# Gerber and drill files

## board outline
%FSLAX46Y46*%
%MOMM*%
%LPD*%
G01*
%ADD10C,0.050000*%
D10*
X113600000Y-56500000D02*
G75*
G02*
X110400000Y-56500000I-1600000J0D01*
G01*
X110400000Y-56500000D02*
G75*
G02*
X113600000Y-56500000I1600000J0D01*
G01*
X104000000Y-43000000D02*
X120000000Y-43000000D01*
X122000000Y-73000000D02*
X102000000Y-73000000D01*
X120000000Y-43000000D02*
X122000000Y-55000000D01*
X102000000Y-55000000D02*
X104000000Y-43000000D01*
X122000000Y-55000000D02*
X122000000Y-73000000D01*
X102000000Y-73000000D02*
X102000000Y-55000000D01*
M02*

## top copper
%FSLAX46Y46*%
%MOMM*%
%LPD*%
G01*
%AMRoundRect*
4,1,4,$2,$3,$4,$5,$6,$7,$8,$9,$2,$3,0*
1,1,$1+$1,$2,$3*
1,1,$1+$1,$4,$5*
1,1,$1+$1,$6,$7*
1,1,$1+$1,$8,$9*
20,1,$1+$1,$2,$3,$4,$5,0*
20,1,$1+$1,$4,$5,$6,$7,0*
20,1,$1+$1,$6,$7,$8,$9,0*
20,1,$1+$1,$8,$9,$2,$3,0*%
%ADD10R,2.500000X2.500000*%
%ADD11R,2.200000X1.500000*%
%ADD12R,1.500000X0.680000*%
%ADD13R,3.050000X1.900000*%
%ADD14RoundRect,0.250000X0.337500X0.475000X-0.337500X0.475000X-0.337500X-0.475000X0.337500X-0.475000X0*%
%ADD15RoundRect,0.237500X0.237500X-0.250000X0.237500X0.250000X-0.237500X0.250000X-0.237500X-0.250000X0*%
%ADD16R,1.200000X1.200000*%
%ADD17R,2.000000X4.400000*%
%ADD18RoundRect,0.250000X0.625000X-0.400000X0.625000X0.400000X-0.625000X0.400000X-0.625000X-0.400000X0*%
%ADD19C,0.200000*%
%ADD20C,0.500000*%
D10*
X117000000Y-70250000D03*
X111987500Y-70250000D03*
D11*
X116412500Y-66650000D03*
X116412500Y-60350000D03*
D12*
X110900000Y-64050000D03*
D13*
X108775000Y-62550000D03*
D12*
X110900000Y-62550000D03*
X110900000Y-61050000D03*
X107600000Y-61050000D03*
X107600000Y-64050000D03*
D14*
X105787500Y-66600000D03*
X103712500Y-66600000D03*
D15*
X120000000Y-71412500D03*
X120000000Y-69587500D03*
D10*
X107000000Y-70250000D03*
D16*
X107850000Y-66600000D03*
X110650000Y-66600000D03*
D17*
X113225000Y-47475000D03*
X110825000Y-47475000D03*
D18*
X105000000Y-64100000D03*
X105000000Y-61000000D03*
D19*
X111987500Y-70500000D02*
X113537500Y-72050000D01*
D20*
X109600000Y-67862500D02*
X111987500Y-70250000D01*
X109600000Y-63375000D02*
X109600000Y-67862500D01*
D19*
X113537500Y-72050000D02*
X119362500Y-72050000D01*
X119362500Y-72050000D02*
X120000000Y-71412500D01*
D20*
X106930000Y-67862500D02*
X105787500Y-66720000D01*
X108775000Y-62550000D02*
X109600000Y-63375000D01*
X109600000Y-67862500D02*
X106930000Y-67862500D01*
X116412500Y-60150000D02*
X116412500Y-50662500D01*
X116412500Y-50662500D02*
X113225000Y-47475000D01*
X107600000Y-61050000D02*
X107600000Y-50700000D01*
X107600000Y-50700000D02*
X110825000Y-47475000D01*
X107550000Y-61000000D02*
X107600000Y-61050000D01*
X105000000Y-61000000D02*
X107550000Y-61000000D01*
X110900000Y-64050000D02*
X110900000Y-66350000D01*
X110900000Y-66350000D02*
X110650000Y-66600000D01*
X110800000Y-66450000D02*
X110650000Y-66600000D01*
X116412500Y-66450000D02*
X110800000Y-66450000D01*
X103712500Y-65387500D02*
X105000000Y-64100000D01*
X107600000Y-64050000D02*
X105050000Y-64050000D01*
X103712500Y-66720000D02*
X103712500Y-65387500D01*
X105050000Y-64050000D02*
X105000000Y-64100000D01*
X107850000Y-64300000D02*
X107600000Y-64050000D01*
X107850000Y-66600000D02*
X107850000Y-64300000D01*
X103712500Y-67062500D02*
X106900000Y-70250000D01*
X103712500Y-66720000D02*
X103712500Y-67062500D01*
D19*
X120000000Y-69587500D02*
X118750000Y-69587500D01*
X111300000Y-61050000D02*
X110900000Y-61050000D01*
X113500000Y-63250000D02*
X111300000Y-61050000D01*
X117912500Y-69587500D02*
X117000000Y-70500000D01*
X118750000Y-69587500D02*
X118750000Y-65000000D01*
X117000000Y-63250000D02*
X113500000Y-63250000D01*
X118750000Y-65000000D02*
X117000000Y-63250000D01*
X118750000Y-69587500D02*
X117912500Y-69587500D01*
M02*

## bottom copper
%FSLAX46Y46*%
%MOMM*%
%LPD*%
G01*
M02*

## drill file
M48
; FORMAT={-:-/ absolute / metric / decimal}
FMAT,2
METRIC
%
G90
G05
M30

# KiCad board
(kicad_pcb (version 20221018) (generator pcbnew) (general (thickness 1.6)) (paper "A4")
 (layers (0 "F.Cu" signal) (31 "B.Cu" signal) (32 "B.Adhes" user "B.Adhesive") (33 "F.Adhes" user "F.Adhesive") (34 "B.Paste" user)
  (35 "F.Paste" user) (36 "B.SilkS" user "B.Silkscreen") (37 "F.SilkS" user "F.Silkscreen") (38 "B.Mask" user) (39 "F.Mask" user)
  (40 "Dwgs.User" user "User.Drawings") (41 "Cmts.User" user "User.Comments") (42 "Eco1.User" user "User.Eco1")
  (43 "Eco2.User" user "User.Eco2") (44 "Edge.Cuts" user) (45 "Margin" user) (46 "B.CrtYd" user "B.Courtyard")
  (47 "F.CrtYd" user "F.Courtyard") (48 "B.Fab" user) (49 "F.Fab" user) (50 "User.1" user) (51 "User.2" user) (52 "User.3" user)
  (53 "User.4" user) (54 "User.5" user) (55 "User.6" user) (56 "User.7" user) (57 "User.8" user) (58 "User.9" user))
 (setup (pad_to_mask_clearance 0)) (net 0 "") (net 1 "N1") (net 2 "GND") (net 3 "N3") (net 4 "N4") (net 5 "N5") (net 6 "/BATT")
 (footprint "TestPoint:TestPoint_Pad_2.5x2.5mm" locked (layer "F.Cu") (at 117 70.25 90)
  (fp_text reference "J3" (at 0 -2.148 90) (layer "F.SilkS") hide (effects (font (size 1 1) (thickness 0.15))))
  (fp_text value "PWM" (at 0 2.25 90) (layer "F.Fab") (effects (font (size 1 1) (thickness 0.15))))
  (pad "1" smd rect locked (at 0 0 90) (size 2.5 2.5) (layers "F.Cu" "F.Mask") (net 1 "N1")))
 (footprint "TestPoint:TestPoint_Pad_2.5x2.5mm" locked (layer "F.Cu") (at 111.9875 70.25 90)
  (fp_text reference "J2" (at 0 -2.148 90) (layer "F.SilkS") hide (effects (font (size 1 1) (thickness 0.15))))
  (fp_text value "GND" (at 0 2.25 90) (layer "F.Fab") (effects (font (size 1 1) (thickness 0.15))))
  (pad "1" smd rect locked (at 0 0 90) (size 2.5 2.5) (layers "F.Cu" "F.Mask") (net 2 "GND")))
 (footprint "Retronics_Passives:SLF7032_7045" (layer "F.Cu") (at 116.4125 63.5 90)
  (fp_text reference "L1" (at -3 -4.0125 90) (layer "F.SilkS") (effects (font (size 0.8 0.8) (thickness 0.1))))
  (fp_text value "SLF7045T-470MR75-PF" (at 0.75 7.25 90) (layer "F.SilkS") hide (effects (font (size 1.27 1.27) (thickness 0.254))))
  (pad "1" smd rect (at -3.15 0 90) (size 1.5 2.2) (layers "F.Cu" "F.Paste" "F.Mask") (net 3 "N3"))
  (pad "2" smd rect (at 3.15 0 90) (size 1.5 2.2) (layers "F.Cu" "F.Paste" "F.Mask") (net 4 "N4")))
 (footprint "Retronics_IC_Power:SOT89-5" (layer "F.Cu") (at 109.25 62.55 90)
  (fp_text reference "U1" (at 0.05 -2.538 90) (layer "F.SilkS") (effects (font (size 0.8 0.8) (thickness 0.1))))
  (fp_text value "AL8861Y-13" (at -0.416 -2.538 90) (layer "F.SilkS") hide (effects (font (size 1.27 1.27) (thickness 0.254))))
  (pad "1" smd rect (at -1.5 1.65 90) (size 0.68 1.5) (layers "F.Cu" "F.Paste" "F.Mask") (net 3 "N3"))
  (pad "2" smd rect (at 0 -0.475 90) (size 1.9 3.05) (layers "F.Cu" "F.Paste" "F.Mask") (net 2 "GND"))
  (pad "2" smd rect (at 0 1.65 90) (size 0.68 1.5) (layers "F.Cu" "F.Paste" "F.Mask") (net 2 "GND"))
  (pad "3" smd rect (at 1.5 1.65 90) (size 0.68 1.5) (layers "F.Cu" "F.Paste" "F.Mask") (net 1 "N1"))
  (pad "4" smd rect (at 1.5 -1.65 90) (size 0.68 1.5) (layers "F.Cu" "F.Paste" "F.Mask") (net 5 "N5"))
  (pad "5" smd rect (at -1.5 -1.65 90) (size 0.68 1.5) (layers "F.Cu" "F.Paste" "F.Mask") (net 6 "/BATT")))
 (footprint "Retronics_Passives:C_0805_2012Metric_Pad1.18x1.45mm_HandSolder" (layer "F.Cu") (at 104.75 66.6 180)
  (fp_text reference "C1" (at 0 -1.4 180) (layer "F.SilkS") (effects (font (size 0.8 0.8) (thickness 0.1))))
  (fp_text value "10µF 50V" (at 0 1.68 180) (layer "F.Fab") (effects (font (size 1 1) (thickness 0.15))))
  (pad "1" smd roundrect (at -1.0375 0 180) (size 1.175 1.45) (layers "F.Cu" "F.Paste" "F.Mask") (roundrect_rratio 0.212766) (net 2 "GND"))
  (pad "2" smd roundrect (at 1.0375 0 180) (size 1.175 1.45) (layers "F.Cu" "F.Paste" "F.Mask") (roundrect_rratio 0.212766) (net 6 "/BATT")))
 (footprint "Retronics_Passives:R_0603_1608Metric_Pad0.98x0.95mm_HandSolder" (layer "F.Cu") (at 120 70.5 90)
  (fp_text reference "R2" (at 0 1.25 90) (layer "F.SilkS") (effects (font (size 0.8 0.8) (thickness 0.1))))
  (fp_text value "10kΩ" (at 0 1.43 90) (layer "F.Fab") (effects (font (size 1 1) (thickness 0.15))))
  (pad "1" smd roundrect (at -0.9125 0 90) (size 0.975 0.95) (layers "F.Cu" "F.Paste" "F.Mask") (roundrect_rratio 0.25) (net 2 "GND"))
  (pad "2" smd roundrect (at 0.9125 0 90) (size 0.975 0.95) (layers "F.Cu" "F.Paste" "F.Mask") (roundrect_rratio 0.25) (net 1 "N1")))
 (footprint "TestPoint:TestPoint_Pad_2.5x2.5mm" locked (layer "F.Cu") (at 107 70.25 90)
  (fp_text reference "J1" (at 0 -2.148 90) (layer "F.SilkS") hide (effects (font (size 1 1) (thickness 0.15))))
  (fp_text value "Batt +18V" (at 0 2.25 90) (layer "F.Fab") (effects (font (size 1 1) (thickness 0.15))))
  (pad "1" smd rect locked (at 0 0 90) (size 2.5 2.5) (layers "F.Cu" "F.Mask") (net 6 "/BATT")))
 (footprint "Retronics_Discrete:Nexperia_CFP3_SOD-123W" (layer "F.Cu") (at 109.25 66.6)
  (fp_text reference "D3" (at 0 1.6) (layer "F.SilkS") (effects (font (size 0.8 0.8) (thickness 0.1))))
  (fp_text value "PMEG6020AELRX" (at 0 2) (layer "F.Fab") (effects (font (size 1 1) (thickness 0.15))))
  (pad "1" smd rect (at -1.4 0) (size 1.2 1.2) (layers "F.Cu" "F.Paste" "F.Mask") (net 6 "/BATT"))
  (pad "2" smd rect (at 1.4 0) (size 1.2 1.2) (layers "F.Cu" "F.Paste" "F.Mask") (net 3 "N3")))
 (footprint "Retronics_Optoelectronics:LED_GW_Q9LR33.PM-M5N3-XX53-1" (layer "F.Cu") (at 112.025 47.475 180)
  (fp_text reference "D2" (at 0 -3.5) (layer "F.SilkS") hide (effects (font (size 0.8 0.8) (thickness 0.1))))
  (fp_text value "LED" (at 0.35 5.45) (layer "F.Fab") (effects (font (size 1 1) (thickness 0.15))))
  (pad "1" smd rect (at -1.2 0 180) (size 2 4.4) (layers "F.Cu" "F.Paste" "F.Mask") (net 4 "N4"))
  (pad "2" smd rect (at 1.2 0 180) (size 2 4.4) (layers "F.Cu" "F.Paste" "F.Mask") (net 5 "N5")))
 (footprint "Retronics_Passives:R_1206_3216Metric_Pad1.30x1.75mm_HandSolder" (layer "F.Cu") (at 105 62.55 90)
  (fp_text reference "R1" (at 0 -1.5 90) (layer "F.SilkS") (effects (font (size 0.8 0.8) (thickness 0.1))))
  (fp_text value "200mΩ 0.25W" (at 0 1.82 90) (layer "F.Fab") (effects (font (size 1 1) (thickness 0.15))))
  (pad "1" smd roundrect (at -1.55 0 90) (size 1.3 1.75) (layers "F.Cu" "F.Paste" "F.Mask") (roundrect_rratio 0.192308) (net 6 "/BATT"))
  (pad "2" smd roundrect (at 1.55 0 90) (size 1.3 1.75) (layers "F.Cu" "F.Paste" "F.Mask") (roundrect_rratio 0.192308) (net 5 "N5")))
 (gr_circle (center 112 56.5) (end 113.6 56.5) (stroke (width 0.05) (type default)) (fill none) (layer "Edge.Cuts"))
 (gr_line (start 104 43) (end 120 43) (stroke (width 0.05) (type default)) (layer "Edge.Cuts"))
 (gr_line (start 122 73) (end 102 73) (stroke (width 0.05) (type default)) (layer "Edge.Cuts"))
 (gr_line (start 120 43) (end 122 55) (stroke (width 0.05) (type default)) (layer "Edge.Cuts"))
 (gr_line (start 102 55) (end 104 43) (stroke (width 0.05) (type default)) (layer "Edge.Cuts"))
 (gr_line (start 122 55) (end 122 73) (stroke (width 0.05) (type default)) (layer "Edge.Cuts"))
 (gr_line (start 102 73) (end 102 55) (stroke (width 0.05) (type default)) (layer "Edge.Cuts"))
 (segment (start 111.9875 70.5) (end 113.5375 72.05) (width 0.2) (layer "F.Cu") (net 2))
 (segment (start 109.6 67.8625) (end 111.9875 70.25) (width 0.5) (layer "F.Cu") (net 2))
 (segment (start 109.6 63.375) (end 109.6 67.8625) (width 0.5) (layer "F.Cu") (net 2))
 (segment (start 113.5375 72.05) (end 119.3625 72.05) (width 0.2) (layer "F.Cu") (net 2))
 (segment (start 119.3625 72.05) (end 120 71.4125) (width 0.2) (layer "F.Cu") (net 2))
 (segment (start 106.93 67.8625) (end 105.7875 66.72) (width 0.5) (layer "F.Cu") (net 2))
 (segment (start 108.775 62.55) (end 109.6 63.375) (width 0.5) (layer "F.Cu") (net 2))
 (segment (start 109.6 67.8625) (end 106.93 67.8625) (width 0.5) (layer "F.Cu") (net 2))
 (segment (start 116.4125 60.15) (end 116.4125 50.6625) (width 0.5) (layer "F.Cu") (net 4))
 (segment (start 116.4125 50.6625) (end 113.225 47.475) (width 0.5) (layer "F.Cu") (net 4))
 (segment (start 107.6 61.05) (end 107.6 50.7) (width 0.5) (layer "F.Cu") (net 5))
 (segment (start 107.6 50.7) (end 110.825 47.475) (width 0.5) (layer "F.Cu") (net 5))
 (segment (start 107.55 61) (end 107.6 61.05) (width 0.5) (layer "F.Cu") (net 5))
 (segment (start 105 61) (end 107.55 61) (width 0.5) (layer "F.Cu") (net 5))
 (segment (start 110.9 64.05) (end 110.9 66.35) (width 0.5) (layer "F.Cu") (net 3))
 (segment (start 110.9 66.35) (end 110.65 66.6) (width 0.5) (layer "F.Cu") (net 3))
 (segment (start 110.8 66.45) (end 110.65 66.6) (width 0.5) (layer "F.Cu") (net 3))
 (segment (start 116.4125 66.45) (end 110.8 66.45) (width 0.5) (layer "F.Cu") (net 3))
 (segment (start 103.7125 65.3875) (end 105 64.1) (width 0.5) (layer "F.Cu") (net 6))
 (segment (start 107.6 64.05) (end 105.05 64.05) (width 0.5) (layer "F.Cu") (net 6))
 (segment (start 103.7125 66.72) (end 103.7125 65.3875) (width 0.5) (layer "F.Cu") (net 6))
 (segment (start 105.05 64.05) (end 105 64.1) (width 0.5) (layer "F.Cu") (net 6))
 (segment (start 107.85 64.3) (end 107.6 64.05) (width 0.5) (layer "F.Cu") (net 6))
 (segment (start 107.85 66.6) (end 107.85 64.3) (width 0.5) (layer "F.Cu") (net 6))
 (segment (start 103.7125 67.0625) (end 106.9 70.25) (width 0.5) (layer "F.Cu") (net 6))
 (segment (start 103.7125 66.72) (end 103.7125 67.0625) (width 0.5) (layer "F.Cu") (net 6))
 (segment (start 120 69.5875) (end 118.75 69.5875) (width 0.2) (layer "F.Cu") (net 1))
 (segment (start 111.3 61.05) (end 110.9 61.05) (width 0.2) (layer "F.Cu") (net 1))
 (segment (start 113.5 63.25) (end 111.3 61.05) (width 0.2) (layer "F.Cu") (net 1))
 (segment (start 117.9125 69.5875) (end 117 70.5) (width 0.2) (layer "F.Cu") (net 1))
 (segment (start 118.75 69.5875) (end 118.75 65) (width 0.2) (layer "F.Cu") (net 1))
 (segment (start 117 63.25) (end 113.5 63.25) (width 0.2) (layer "F.Cu") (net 1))
 (segment (start 118.75 65) (end 117 63.25) (width 0.2) (layer "F.Cu") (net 1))
 (segment (start 118.75 69.5875) (end 117.9125 69.5875) (width 0.2) (layer "F.Cu") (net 1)))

